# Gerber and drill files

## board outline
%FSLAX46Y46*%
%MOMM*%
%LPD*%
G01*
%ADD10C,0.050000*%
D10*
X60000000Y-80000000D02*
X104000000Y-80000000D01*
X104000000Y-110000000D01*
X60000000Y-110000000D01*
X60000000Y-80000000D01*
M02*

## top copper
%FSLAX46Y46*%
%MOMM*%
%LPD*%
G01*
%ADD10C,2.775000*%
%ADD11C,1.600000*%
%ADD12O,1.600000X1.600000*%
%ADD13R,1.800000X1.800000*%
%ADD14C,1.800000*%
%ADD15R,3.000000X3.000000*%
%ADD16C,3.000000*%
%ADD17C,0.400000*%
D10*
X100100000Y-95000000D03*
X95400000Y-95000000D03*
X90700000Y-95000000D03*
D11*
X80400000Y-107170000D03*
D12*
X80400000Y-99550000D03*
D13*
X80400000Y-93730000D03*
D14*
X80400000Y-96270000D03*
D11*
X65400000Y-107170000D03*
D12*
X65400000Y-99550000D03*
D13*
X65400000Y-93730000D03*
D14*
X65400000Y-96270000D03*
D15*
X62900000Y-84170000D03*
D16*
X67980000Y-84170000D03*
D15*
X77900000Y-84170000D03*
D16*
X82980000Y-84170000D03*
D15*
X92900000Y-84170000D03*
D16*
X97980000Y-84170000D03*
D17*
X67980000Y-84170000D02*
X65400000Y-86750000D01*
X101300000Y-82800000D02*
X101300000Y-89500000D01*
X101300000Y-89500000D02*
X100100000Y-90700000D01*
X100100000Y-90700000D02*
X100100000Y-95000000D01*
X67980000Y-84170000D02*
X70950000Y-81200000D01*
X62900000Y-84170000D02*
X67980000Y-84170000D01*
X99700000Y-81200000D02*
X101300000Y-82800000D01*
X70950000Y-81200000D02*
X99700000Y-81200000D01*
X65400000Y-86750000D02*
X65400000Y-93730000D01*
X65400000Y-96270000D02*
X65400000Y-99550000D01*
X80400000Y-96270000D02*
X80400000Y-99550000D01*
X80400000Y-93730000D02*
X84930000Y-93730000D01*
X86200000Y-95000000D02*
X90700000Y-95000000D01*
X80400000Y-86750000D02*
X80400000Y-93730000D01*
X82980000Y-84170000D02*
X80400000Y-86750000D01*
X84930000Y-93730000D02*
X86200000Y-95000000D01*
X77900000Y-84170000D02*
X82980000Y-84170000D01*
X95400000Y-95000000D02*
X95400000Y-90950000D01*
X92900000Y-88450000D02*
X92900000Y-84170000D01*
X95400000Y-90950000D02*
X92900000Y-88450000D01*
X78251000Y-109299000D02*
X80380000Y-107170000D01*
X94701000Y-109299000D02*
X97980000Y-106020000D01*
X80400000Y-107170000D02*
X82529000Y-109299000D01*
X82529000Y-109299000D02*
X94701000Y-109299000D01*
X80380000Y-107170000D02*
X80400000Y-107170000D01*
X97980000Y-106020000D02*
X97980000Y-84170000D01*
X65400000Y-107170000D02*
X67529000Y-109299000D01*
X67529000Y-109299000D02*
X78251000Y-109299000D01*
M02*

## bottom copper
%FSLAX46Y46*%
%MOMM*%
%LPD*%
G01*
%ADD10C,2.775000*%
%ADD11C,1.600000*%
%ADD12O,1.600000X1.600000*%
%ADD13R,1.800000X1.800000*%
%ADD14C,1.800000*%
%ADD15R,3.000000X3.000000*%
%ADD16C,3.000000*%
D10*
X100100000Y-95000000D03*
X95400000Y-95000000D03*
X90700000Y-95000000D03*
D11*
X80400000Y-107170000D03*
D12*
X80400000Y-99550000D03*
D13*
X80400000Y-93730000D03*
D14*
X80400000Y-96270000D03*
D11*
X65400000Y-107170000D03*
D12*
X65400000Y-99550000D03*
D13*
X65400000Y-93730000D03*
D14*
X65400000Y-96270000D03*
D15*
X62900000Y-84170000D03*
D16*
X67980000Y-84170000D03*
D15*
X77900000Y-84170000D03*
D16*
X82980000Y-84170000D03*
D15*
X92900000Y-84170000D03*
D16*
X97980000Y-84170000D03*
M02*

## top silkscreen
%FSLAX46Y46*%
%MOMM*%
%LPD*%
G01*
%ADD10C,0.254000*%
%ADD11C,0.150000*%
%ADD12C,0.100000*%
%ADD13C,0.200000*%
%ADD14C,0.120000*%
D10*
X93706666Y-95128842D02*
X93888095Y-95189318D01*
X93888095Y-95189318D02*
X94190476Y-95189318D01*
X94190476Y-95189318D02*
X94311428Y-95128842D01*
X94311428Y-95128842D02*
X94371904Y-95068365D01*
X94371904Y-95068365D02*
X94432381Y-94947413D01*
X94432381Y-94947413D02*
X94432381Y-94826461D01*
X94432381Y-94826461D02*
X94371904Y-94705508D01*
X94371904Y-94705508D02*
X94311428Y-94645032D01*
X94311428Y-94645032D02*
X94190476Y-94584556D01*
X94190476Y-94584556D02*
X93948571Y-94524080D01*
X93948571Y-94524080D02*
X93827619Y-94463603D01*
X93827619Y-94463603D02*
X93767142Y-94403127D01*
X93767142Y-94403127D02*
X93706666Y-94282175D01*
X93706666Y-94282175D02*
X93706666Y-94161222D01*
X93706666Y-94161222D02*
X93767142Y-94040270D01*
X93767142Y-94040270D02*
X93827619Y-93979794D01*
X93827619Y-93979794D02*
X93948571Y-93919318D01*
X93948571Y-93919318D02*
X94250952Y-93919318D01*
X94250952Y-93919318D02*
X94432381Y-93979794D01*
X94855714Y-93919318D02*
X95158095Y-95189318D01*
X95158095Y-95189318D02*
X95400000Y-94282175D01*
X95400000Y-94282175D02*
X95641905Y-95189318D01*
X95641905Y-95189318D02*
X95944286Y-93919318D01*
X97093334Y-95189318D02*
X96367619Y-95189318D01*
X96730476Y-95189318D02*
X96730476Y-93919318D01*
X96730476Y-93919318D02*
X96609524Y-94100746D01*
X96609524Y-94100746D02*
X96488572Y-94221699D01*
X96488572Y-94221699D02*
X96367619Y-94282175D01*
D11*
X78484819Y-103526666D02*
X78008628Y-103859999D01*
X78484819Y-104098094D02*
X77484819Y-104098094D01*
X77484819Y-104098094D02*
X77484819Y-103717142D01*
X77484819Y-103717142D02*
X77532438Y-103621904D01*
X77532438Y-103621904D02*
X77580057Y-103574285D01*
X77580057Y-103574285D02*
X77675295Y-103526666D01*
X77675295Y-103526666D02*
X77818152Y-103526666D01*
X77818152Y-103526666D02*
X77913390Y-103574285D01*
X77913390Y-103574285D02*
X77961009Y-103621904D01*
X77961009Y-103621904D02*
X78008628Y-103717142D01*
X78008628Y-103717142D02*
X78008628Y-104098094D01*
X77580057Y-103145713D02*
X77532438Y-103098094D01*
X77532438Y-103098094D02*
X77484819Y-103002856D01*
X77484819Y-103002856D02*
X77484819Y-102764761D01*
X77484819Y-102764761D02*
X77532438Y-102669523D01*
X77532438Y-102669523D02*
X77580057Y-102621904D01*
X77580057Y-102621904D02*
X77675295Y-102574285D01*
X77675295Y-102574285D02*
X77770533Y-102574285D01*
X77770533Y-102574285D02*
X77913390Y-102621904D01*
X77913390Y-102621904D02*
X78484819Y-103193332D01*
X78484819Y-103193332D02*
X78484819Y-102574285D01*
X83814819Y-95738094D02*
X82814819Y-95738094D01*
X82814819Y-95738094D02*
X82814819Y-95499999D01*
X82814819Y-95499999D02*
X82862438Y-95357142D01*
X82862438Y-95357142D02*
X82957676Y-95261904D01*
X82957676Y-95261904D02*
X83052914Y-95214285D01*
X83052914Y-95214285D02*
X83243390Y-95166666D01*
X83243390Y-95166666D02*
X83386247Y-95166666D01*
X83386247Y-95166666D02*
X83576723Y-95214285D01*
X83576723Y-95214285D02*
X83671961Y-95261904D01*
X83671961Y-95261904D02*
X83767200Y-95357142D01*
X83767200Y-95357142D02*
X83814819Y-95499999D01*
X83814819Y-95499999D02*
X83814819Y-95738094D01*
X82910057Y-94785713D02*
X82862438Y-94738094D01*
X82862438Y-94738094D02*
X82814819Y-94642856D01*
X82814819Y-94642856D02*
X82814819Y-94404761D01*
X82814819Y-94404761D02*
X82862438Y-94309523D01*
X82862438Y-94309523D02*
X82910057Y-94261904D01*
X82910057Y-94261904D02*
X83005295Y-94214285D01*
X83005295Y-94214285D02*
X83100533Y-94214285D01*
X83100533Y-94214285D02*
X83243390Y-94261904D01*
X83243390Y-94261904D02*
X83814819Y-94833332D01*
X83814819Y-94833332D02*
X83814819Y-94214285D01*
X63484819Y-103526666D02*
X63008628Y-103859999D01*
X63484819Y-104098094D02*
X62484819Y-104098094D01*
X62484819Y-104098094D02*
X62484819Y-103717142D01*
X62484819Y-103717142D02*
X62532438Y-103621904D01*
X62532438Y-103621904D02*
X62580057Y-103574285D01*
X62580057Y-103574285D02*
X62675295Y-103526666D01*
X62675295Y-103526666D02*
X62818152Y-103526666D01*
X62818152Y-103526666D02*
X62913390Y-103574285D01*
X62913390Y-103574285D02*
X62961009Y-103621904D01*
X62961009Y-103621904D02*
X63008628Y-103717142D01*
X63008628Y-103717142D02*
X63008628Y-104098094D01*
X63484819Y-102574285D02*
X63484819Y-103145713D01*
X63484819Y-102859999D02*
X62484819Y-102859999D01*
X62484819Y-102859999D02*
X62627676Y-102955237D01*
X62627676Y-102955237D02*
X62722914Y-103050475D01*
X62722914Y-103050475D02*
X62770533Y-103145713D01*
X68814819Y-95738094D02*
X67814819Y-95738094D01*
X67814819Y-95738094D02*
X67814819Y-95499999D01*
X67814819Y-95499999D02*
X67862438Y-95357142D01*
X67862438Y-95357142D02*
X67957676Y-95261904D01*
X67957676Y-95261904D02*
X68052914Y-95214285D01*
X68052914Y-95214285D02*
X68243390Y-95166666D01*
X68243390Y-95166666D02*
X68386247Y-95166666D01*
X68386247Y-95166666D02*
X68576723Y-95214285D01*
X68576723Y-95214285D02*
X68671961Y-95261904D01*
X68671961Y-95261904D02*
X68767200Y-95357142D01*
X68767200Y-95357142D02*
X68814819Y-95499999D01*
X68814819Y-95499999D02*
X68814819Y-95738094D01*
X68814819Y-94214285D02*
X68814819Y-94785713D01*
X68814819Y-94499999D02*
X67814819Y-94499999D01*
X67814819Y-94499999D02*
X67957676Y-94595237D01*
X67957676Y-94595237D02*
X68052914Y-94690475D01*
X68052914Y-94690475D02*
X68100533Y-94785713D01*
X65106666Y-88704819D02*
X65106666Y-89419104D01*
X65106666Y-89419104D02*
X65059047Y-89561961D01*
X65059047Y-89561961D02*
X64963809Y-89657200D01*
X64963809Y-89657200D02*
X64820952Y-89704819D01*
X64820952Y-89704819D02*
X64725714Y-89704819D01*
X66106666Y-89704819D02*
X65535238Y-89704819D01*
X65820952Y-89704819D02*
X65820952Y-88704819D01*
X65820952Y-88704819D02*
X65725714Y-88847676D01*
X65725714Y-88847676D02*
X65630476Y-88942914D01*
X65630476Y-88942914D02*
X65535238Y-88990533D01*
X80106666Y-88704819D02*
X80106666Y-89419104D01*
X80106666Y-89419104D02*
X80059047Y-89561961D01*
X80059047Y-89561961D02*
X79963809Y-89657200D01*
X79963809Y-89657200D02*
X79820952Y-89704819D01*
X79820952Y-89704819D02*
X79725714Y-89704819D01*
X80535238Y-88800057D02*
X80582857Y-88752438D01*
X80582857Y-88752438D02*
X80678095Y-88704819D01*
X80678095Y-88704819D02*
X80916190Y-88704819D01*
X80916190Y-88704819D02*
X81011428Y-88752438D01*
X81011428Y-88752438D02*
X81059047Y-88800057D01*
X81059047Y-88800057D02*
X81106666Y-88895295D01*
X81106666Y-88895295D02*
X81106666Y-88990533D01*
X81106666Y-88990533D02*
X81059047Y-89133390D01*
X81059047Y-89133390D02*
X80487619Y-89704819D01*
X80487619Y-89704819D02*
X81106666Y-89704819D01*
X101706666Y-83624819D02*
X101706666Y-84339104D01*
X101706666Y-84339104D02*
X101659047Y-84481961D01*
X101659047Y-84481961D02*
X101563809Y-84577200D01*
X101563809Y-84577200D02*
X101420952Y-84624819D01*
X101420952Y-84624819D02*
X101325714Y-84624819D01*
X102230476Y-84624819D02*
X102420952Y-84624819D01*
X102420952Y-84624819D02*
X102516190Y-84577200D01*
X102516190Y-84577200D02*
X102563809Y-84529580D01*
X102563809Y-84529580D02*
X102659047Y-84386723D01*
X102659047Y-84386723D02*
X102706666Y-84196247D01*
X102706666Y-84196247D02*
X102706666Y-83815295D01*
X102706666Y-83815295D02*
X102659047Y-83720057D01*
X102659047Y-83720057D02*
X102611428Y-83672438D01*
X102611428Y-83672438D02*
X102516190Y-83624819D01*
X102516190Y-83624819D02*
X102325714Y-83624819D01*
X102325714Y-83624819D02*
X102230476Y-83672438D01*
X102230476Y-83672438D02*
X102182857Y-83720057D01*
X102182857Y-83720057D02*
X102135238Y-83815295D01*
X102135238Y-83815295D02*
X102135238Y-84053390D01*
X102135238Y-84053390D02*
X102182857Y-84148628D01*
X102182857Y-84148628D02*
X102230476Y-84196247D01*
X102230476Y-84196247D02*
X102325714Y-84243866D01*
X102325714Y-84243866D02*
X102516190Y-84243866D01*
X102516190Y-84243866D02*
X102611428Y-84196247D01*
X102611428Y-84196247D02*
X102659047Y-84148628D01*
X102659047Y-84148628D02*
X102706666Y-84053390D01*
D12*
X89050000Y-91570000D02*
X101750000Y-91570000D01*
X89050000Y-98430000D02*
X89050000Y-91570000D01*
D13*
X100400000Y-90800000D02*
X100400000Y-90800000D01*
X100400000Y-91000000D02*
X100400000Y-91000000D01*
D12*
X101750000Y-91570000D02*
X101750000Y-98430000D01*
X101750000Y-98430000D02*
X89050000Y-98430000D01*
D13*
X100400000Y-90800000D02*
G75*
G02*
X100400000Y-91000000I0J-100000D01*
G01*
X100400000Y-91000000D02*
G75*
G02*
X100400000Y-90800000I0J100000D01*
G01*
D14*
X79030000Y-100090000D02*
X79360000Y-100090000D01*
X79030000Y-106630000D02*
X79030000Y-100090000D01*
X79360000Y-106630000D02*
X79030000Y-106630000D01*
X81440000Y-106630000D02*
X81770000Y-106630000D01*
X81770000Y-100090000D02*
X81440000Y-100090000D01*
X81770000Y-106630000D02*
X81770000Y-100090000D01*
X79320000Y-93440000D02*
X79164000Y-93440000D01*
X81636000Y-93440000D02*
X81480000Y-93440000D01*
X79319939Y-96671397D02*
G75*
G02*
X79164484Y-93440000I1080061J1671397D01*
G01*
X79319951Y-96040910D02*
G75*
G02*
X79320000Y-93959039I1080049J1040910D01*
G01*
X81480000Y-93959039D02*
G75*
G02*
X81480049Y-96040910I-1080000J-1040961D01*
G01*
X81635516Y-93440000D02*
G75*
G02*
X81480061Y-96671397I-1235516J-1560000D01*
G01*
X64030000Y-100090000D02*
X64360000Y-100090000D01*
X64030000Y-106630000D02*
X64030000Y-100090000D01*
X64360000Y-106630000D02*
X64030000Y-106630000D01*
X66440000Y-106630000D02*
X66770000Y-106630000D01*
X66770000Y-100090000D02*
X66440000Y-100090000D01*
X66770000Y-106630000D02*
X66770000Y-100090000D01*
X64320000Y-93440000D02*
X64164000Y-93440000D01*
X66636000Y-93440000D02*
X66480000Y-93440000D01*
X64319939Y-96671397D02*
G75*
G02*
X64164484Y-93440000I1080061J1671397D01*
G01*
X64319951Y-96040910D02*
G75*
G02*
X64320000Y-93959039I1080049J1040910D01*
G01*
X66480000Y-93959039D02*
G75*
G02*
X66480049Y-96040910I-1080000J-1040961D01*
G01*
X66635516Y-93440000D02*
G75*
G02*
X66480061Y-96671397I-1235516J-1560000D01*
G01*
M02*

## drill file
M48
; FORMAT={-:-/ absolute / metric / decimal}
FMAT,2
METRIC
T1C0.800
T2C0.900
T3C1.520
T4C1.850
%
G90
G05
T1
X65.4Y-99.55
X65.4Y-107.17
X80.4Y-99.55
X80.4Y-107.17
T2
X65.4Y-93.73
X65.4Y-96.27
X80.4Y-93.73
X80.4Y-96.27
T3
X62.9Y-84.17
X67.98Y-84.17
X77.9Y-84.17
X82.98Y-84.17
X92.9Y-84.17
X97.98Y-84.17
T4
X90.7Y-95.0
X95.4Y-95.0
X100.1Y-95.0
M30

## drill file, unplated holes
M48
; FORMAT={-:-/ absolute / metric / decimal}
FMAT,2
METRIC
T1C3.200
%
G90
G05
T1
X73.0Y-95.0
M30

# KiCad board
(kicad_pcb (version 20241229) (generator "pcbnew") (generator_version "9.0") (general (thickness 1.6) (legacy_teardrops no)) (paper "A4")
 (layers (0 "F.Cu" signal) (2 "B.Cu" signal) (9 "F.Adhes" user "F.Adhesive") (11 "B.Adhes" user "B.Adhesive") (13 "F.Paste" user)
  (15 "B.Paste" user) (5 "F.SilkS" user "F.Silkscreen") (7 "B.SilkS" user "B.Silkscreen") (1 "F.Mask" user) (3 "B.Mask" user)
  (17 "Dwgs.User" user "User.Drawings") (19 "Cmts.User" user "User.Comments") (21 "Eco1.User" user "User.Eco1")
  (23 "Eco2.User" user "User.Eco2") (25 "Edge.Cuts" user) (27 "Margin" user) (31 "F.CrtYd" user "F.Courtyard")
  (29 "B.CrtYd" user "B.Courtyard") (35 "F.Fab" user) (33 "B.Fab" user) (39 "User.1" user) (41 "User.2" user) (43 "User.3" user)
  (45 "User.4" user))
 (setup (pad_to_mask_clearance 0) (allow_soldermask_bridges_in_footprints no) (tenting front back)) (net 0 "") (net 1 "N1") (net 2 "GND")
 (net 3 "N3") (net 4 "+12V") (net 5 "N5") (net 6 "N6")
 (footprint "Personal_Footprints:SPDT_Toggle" (layer "F.Cu") (at 100.1 95 180)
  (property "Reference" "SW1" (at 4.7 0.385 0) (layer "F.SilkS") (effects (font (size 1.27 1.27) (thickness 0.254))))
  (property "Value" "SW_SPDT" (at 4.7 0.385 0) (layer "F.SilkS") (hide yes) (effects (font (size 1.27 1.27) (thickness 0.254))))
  (fp_line (start 11.05 3.43) (end -1.65 3.43) (stroke (width 0.1) (type solid)) (layer "F.SilkS"))
  (fp_line (start 11.05 -3.43) (end 11.05 3.43) (stroke (width 0.1) (type solid)) (layer "F.SilkS"))
  (fp_line (start -0.3 4.2) (end -0.3 4.2) (stroke (width 0.2) (type solid)) (layer "F.SilkS"))
  (fp_line (start -0.3 4) (end -0.3 4) (stroke (width 0.2) (type solid)) (layer "F.SilkS"))
  (fp_line (start -1.65 3.43) (end -1.65 -3.43) (stroke (width 0.1) (type solid)) (layer "F.SilkS"))
  (fp_line (start -1.65 -3.43) (end 11.05 -3.43) (stroke (width 0.1) (type solid)) (layer "F.SilkS"))
  (fp_arc (start -0.3 4.2) (mid -0.4 4.1) (end -0.3 4) (stroke (width 0.2) (type solid)) (layer "F.SilkS"))
  (fp_arc (start -0.3 4) (mid -0.2 4.1) (end -0.3 4.2) (stroke (width 0.2) (type solid)) (layer "F.SilkS"))
  (pad "1" thru_hole circle (at 0 0 180) (size 2.775 2.775) (drill 1.85) (layers "*.Cu" "*.Mask") (remove_unused_layers no) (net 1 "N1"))
  (pad "2" thru_hole circle (at 4.7 0 180) (size 2.775 2.775) (drill 1.85) (layers "*.Cu" "*.Mask") (remove_unused_layers no) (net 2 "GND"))
  (pad "3" thru_hole circle (at 9.4 0 180) (size 2.775 2.775) (drill 1.85) (layers "*.Cu" "*.Mask") (remove_unused_layers no) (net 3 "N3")))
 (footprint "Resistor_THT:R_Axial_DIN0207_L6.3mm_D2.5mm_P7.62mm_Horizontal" (layer "F.Cu") (at 80.4 107.17 90)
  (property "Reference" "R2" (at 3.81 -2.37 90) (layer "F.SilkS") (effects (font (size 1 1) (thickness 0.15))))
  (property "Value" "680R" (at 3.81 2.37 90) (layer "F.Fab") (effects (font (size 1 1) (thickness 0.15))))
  (fp_line (start 7.08 -1.37) (end 7.08 -1.04) (stroke (width 0.12) (type solid)) (layer "F.SilkS"))
  (fp_line (start 0.54 -1.37) (end 7.08 -1.37) (stroke (width 0.12) (type solid)) (layer "F.SilkS"))
  (fp_line (start 0.54 -1.04) (end 0.54 -1.37) (stroke (width 0.12) (type solid)) (layer "F.SilkS"))
  (fp_line (start 0.54 1.04) (end 0.54 1.37) (stroke (width 0.12) (type solid)) (layer "F.SilkS"))
  (fp_line (start 7.08 1.37) (end 7.08 1.04) (stroke (width 0.12) (type solid)) (layer "F.SilkS"))
  (fp_line (start 0.54 1.37) (end 7.08 1.37) (stroke (width 0.12) (type solid)) (layer "F.SilkS"))
  (pad "1" thru_hole circle (at 0 0 90) (size 1.6 1.6) (drill 0.8) (layers "*.Cu" "*.Mask") (remove_unused_layers no) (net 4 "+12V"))
  (pad "2" thru_hole oval (at 7.62 0 90) (size 1.6 1.6) (drill 0.8) (layers "*.Cu" "*.Mask") (remove_unused_layers no) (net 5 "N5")))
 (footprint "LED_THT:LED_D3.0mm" (layer "F.Cu") (at 80.4 93.73 -90)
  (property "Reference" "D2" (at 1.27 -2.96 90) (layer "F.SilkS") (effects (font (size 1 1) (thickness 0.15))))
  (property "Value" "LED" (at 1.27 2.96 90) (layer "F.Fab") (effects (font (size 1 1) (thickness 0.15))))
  (fp_line (start -0.29 1.08) (end -0.29 1.236) (stroke (width 0.12) (type solid)) (layer "F.SilkS"))
  (fp_line (start -0.29 -1.236) (end -0.29 -1.08) (stroke (width 0.12) (type solid)) (layer "F.SilkS"))
  (fp_arc (start 2.941397 1.080061) (mid 1.365624 1.987701) (end -0.29 1.235516) (stroke (width 0.12) (type solid)) (layer "F.SilkS"))
  (fp_arc (start 2.31091 1.080049) (mid 1.269964 1.5) (end 0.229039 1.08) (stroke (width 0.12) (type solid)) (layer "F.SilkS"))
  (fp_arc (start 0.229039 -1.08) (mid 1.269964 -1.5) (end 2.31091 -1.080049) (stroke (width 0.12) (type solid)) (layer "F.SilkS"))
  (fp_arc (start -0.29 -1.235516) (mid 1.365624 -1.987701) (end 2.941397 -1.080061) (stroke (width 0.12) (type solid)) (layer "F.SilkS"))
  (pad "1" thru_hole rect (at 0 0 270) (size 1.8 1.8) (drill 0.9) (layers "*.Cu" "*.Mask") (remove_unused_layers no) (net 3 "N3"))
  (pad "2" thru_hole circle (at 2.54 0 270) (size 1.8 1.8) (drill 0.9) (layers "*.Cu" "*.Mask") (remove_unused_layers no) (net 5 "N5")))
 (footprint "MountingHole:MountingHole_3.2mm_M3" (layer "F.Cu") (at 73 95)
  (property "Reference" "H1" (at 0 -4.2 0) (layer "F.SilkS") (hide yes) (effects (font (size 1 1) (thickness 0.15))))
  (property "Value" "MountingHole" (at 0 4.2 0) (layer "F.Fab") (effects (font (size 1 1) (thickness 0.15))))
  (pad "" np_thru_hole circle (at 0 0) (size 3.2 3.2) (drill 3.2) (layers "*.Cu" "*.Mask")))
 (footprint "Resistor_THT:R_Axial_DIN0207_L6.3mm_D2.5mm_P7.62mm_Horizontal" (layer "F.Cu") (at 65.4 107.17 90)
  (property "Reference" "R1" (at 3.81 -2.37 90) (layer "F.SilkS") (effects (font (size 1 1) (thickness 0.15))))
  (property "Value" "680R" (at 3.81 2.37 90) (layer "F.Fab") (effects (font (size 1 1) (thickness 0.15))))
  (fp_line (start 7.08 -1.37) (end 7.08 -1.04) (stroke (width 0.12) (type solid)) (layer "F.SilkS"))
  (fp_line (start 0.54 -1.37) (end 7.08 -1.37) (stroke (width 0.12) (type solid)) (layer "F.SilkS"))
  (fp_line (start 0.54 -1.04) (end 0.54 -1.37) (stroke (width 0.12) (type solid)) (layer "F.SilkS"))
  (fp_line (start 0.54 1.04) (end 0.54 1.37) (stroke (width 0.12) (type solid)) (layer "F.SilkS"))
  (fp_line (start 7.08 1.37) (end 7.08 1.04) (stroke (width 0.12) (type solid)) (layer "F.SilkS"))
  (fp_line (start 0.54 1.37) (end 7.08 1.37) (stroke (width 0.12) (type solid)) (layer "F.SilkS"))
  (pad "1" thru_hole circle (at 0 0 90) (size 1.6 1.6) (drill 0.8) (layers "*.Cu" "*.Mask") (remove_unused_layers no) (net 4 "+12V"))
  (pad "2" thru_hole oval (at 7.62 0 90) (size 1.6 1.6) (drill 0.8) (layers "*.Cu" "*.Mask") (remove_unused_layers no) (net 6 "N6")))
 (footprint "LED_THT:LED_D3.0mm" (layer "F.Cu") (at 65.4 93.73 -90)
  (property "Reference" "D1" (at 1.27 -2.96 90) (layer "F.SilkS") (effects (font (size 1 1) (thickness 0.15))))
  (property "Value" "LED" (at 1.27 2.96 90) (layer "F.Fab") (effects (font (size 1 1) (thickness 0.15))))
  (fp_line (start -0.29 1.08) (end -0.29 1.236) (stroke (width 0.12) (type solid)) (layer "F.SilkS"))
  (fp_line (start -0.29 -1.236) (end -0.29 -1.08) (stroke (width 0.12) (type solid)) (layer "F.SilkS"))
  (fp_arc (start 2.941397 1.080061) (mid 1.365624 1.987701) (end -0.29 1.235516) (stroke (width 0.12) (type solid)) (layer "F.SilkS"))
  (fp_arc (start 2.31091 1.080049) (mid 1.269964 1.5) (end 0.229039 1.08) (stroke (width 0.12) (type solid)) (layer "F.SilkS"))
  (fp_arc (start 0.229039 -1.08) (mid 1.269964 -1.5) (end 2.31091 -1.080049) (stroke (width 0.12) (type solid)) (layer "F.SilkS"))
  (fp_arc (start -0.29 -1.235516) (mid 1.365624 -1.987701) (end 2.941397 -1.080061) (stroke (width 0.12) (type solid)) (layer "F.SilkS"))
  (pad "1" thru_hole rect (at 0 0 270) (size 1.8 1.8) (drill 0.9) (layers "*.Cu" "*.Mask") (remove_unused_layers no) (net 1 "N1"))
  (pad "2" thru_hole circle (at 2.54 0 270) (size 1.8 1.8) (drill 0.9) (layers "*.Cu" "*.Mask") (remove_unused_layers no) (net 6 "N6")))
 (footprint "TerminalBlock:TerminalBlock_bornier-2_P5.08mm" (layer "B.Cu") (at 62.9 84.17)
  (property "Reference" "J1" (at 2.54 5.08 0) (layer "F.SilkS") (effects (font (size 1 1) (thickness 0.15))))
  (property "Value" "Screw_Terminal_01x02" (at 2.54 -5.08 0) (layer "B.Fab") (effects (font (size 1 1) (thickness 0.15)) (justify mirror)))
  (pad "1" thru_hole rect (at 0 0) (size 3 3) (drill 1.52) (layers "*.Cu" "*.Mask") (remove_unused_layers no) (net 1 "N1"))
  (pad "2" thru_hole circle (at 5.08 0) (size 3 3) (drill 1.52) (layers "*.Cu" "*.Mask") (remove_unused_layers no) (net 1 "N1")))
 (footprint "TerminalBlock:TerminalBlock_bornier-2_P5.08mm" (layer "B.Cu") (at 77.9 84.17)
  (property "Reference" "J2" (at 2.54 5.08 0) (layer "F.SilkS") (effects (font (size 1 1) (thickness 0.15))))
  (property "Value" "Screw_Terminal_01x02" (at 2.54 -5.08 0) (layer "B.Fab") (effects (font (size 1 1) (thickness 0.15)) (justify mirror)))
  (pad "1" thru_hole rect (at 0 0) (size 3 3) (drill 1.52) (layers "*.Cu" "*.Mask") (remove_unused_layers no) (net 3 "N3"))
  (pad "2" thru_hole circle (at 5.08 0) (size 3 3) (drill 1.52) (layers "*.Cu" "*.Mask") (remove_unused_layers no) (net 3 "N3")))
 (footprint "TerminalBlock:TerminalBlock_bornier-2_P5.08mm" (layer "B.Cu") (at 92.9 84.17)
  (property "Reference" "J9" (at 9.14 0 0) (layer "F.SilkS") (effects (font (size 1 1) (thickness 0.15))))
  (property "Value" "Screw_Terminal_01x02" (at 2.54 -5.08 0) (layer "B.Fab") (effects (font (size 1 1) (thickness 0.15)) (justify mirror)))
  (pad "1" thru_hole rect (at 0 0) (size 3 3) (drill 1.52) (layers "*.Cu" "*.Mask") (remove_unused_layers no) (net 2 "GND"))
  (pad "2" thru_hole circle (at 5.08 0) (size 3 3) (drill 1.52) (layers "*.Cu" "*.Mask") (remove_unused_layers no) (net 4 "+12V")))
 (gr_rect (start 60 80) (end 104 110) (stroke (width 0.05) (type solid)) (fill no) (layer "Edge.Cuts"))
 (segment (start 67.98 84.17) (end 65.4 86.75) (width 0.4) (layer "F.Cu") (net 1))
 (segment (start 101.3 82.8) (end 101.3 89.5) (width 0.4) (layer "F.Cu") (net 1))
 (segment (start 101.3 89.5) (end 100.1 90.7) (width 0.4) (layer "F.Cu") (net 1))
 (segment (start 100.1 90.7) (end 100.1 95) (width 0.4) (layer "F.Cu") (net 1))
 (segment (start 67.98 84.17) (end 70.95 81.2) (width 0.4) (layer "F.Cu") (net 1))
 (segment (start 62.9 84.17) (end 67.98 84.17) (width 0.4) (layer "F.Cu") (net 1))
 (segment (start 99.7 81.2) (end 101.3 82.8) (width 0.4) (layer "F.Cu") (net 1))
 (segment (start 70.95 81.2) (end 99.7 81.2) (width 0.4) (layer "F.Cu") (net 1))
 (segment (start 65.4 86.75) (end 65.4 93.73) (width 0.4) (layer "F.Cu") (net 1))
 (segment (start 65.4 96.27) (end 65.4 99.55) (width 0.4) (layer "F.Cu") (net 6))
 (segment (start 80.4 96.27) (end 80.4 99.55) (width 0.4) (layer "F.Cu") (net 5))
 (segment (start 80.4 93.73) (end 84.93 93.73) (width 0.4) (layer "F.Cu") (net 3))
 (segment (start 86.2 95) (end 90.7 95) (width 0.4) (layer "F.Cu") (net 3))
 (segment (start 80.4 86.75) (end 80.4 93.73) (width 0.4) (layer "F.Cu") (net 3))
 (segment (start 82.98 84.17) (end 80.4 86.75) (width 0.4) (layer "F.Cu") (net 3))
 (segment (start 84.93 93.73) (end 86.2 95) (width 0.4) (layer "F.Cu") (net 3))
 (segment (start 77.9 84.17) (end 82.98 84.17) (width 0.4) (layer "F.Cu") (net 3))
 (segment (start 95.4 95) (end 95.4 90.95) (width 0.4) (layer "F.Cu") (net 2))
 (segment (start 92.9 88.45) (end 92.9 84.17) (width 0.4) (layer "F.Cu") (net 2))
 (segment (start 95.4 90.95) (end 92.9 88.45) (width 0.4) (layer "F.Cu") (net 2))
 (segment (start 78.251 109.299) (end 80.38 107.17) (width 0.4) (layer "F.Cu") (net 4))
 (segment (start 94.701 109.299) (end 97.98 106.02) (width 0.4) (layer "F.Cu") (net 4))
 (segment (start 80.4 107.17) (end 82.529 109.299) (width 0.4) (layer "F.Cu") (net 4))
 (segment (start 82.529 109.299) (end 94.701 109.299) (width 0.4) (layer "F.Cu") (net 4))
 (segment (start 80.38 107.17) (end 80.4 107.17) (width 0.4) (layer "F.Cu") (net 4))
 (segment (start 97.98 106.02) (end 97.98 84.17) (width 0.4) (layer "F.Cu") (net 4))
 (segment (start 65.4 107.17) (end 67.529 109.299) (width 0.4) (layer "F.Cu") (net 4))
 (segment (start 67.529 109.299) (end 78.251 109.299) (width 0.4) (layer "F.Cu") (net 4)))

